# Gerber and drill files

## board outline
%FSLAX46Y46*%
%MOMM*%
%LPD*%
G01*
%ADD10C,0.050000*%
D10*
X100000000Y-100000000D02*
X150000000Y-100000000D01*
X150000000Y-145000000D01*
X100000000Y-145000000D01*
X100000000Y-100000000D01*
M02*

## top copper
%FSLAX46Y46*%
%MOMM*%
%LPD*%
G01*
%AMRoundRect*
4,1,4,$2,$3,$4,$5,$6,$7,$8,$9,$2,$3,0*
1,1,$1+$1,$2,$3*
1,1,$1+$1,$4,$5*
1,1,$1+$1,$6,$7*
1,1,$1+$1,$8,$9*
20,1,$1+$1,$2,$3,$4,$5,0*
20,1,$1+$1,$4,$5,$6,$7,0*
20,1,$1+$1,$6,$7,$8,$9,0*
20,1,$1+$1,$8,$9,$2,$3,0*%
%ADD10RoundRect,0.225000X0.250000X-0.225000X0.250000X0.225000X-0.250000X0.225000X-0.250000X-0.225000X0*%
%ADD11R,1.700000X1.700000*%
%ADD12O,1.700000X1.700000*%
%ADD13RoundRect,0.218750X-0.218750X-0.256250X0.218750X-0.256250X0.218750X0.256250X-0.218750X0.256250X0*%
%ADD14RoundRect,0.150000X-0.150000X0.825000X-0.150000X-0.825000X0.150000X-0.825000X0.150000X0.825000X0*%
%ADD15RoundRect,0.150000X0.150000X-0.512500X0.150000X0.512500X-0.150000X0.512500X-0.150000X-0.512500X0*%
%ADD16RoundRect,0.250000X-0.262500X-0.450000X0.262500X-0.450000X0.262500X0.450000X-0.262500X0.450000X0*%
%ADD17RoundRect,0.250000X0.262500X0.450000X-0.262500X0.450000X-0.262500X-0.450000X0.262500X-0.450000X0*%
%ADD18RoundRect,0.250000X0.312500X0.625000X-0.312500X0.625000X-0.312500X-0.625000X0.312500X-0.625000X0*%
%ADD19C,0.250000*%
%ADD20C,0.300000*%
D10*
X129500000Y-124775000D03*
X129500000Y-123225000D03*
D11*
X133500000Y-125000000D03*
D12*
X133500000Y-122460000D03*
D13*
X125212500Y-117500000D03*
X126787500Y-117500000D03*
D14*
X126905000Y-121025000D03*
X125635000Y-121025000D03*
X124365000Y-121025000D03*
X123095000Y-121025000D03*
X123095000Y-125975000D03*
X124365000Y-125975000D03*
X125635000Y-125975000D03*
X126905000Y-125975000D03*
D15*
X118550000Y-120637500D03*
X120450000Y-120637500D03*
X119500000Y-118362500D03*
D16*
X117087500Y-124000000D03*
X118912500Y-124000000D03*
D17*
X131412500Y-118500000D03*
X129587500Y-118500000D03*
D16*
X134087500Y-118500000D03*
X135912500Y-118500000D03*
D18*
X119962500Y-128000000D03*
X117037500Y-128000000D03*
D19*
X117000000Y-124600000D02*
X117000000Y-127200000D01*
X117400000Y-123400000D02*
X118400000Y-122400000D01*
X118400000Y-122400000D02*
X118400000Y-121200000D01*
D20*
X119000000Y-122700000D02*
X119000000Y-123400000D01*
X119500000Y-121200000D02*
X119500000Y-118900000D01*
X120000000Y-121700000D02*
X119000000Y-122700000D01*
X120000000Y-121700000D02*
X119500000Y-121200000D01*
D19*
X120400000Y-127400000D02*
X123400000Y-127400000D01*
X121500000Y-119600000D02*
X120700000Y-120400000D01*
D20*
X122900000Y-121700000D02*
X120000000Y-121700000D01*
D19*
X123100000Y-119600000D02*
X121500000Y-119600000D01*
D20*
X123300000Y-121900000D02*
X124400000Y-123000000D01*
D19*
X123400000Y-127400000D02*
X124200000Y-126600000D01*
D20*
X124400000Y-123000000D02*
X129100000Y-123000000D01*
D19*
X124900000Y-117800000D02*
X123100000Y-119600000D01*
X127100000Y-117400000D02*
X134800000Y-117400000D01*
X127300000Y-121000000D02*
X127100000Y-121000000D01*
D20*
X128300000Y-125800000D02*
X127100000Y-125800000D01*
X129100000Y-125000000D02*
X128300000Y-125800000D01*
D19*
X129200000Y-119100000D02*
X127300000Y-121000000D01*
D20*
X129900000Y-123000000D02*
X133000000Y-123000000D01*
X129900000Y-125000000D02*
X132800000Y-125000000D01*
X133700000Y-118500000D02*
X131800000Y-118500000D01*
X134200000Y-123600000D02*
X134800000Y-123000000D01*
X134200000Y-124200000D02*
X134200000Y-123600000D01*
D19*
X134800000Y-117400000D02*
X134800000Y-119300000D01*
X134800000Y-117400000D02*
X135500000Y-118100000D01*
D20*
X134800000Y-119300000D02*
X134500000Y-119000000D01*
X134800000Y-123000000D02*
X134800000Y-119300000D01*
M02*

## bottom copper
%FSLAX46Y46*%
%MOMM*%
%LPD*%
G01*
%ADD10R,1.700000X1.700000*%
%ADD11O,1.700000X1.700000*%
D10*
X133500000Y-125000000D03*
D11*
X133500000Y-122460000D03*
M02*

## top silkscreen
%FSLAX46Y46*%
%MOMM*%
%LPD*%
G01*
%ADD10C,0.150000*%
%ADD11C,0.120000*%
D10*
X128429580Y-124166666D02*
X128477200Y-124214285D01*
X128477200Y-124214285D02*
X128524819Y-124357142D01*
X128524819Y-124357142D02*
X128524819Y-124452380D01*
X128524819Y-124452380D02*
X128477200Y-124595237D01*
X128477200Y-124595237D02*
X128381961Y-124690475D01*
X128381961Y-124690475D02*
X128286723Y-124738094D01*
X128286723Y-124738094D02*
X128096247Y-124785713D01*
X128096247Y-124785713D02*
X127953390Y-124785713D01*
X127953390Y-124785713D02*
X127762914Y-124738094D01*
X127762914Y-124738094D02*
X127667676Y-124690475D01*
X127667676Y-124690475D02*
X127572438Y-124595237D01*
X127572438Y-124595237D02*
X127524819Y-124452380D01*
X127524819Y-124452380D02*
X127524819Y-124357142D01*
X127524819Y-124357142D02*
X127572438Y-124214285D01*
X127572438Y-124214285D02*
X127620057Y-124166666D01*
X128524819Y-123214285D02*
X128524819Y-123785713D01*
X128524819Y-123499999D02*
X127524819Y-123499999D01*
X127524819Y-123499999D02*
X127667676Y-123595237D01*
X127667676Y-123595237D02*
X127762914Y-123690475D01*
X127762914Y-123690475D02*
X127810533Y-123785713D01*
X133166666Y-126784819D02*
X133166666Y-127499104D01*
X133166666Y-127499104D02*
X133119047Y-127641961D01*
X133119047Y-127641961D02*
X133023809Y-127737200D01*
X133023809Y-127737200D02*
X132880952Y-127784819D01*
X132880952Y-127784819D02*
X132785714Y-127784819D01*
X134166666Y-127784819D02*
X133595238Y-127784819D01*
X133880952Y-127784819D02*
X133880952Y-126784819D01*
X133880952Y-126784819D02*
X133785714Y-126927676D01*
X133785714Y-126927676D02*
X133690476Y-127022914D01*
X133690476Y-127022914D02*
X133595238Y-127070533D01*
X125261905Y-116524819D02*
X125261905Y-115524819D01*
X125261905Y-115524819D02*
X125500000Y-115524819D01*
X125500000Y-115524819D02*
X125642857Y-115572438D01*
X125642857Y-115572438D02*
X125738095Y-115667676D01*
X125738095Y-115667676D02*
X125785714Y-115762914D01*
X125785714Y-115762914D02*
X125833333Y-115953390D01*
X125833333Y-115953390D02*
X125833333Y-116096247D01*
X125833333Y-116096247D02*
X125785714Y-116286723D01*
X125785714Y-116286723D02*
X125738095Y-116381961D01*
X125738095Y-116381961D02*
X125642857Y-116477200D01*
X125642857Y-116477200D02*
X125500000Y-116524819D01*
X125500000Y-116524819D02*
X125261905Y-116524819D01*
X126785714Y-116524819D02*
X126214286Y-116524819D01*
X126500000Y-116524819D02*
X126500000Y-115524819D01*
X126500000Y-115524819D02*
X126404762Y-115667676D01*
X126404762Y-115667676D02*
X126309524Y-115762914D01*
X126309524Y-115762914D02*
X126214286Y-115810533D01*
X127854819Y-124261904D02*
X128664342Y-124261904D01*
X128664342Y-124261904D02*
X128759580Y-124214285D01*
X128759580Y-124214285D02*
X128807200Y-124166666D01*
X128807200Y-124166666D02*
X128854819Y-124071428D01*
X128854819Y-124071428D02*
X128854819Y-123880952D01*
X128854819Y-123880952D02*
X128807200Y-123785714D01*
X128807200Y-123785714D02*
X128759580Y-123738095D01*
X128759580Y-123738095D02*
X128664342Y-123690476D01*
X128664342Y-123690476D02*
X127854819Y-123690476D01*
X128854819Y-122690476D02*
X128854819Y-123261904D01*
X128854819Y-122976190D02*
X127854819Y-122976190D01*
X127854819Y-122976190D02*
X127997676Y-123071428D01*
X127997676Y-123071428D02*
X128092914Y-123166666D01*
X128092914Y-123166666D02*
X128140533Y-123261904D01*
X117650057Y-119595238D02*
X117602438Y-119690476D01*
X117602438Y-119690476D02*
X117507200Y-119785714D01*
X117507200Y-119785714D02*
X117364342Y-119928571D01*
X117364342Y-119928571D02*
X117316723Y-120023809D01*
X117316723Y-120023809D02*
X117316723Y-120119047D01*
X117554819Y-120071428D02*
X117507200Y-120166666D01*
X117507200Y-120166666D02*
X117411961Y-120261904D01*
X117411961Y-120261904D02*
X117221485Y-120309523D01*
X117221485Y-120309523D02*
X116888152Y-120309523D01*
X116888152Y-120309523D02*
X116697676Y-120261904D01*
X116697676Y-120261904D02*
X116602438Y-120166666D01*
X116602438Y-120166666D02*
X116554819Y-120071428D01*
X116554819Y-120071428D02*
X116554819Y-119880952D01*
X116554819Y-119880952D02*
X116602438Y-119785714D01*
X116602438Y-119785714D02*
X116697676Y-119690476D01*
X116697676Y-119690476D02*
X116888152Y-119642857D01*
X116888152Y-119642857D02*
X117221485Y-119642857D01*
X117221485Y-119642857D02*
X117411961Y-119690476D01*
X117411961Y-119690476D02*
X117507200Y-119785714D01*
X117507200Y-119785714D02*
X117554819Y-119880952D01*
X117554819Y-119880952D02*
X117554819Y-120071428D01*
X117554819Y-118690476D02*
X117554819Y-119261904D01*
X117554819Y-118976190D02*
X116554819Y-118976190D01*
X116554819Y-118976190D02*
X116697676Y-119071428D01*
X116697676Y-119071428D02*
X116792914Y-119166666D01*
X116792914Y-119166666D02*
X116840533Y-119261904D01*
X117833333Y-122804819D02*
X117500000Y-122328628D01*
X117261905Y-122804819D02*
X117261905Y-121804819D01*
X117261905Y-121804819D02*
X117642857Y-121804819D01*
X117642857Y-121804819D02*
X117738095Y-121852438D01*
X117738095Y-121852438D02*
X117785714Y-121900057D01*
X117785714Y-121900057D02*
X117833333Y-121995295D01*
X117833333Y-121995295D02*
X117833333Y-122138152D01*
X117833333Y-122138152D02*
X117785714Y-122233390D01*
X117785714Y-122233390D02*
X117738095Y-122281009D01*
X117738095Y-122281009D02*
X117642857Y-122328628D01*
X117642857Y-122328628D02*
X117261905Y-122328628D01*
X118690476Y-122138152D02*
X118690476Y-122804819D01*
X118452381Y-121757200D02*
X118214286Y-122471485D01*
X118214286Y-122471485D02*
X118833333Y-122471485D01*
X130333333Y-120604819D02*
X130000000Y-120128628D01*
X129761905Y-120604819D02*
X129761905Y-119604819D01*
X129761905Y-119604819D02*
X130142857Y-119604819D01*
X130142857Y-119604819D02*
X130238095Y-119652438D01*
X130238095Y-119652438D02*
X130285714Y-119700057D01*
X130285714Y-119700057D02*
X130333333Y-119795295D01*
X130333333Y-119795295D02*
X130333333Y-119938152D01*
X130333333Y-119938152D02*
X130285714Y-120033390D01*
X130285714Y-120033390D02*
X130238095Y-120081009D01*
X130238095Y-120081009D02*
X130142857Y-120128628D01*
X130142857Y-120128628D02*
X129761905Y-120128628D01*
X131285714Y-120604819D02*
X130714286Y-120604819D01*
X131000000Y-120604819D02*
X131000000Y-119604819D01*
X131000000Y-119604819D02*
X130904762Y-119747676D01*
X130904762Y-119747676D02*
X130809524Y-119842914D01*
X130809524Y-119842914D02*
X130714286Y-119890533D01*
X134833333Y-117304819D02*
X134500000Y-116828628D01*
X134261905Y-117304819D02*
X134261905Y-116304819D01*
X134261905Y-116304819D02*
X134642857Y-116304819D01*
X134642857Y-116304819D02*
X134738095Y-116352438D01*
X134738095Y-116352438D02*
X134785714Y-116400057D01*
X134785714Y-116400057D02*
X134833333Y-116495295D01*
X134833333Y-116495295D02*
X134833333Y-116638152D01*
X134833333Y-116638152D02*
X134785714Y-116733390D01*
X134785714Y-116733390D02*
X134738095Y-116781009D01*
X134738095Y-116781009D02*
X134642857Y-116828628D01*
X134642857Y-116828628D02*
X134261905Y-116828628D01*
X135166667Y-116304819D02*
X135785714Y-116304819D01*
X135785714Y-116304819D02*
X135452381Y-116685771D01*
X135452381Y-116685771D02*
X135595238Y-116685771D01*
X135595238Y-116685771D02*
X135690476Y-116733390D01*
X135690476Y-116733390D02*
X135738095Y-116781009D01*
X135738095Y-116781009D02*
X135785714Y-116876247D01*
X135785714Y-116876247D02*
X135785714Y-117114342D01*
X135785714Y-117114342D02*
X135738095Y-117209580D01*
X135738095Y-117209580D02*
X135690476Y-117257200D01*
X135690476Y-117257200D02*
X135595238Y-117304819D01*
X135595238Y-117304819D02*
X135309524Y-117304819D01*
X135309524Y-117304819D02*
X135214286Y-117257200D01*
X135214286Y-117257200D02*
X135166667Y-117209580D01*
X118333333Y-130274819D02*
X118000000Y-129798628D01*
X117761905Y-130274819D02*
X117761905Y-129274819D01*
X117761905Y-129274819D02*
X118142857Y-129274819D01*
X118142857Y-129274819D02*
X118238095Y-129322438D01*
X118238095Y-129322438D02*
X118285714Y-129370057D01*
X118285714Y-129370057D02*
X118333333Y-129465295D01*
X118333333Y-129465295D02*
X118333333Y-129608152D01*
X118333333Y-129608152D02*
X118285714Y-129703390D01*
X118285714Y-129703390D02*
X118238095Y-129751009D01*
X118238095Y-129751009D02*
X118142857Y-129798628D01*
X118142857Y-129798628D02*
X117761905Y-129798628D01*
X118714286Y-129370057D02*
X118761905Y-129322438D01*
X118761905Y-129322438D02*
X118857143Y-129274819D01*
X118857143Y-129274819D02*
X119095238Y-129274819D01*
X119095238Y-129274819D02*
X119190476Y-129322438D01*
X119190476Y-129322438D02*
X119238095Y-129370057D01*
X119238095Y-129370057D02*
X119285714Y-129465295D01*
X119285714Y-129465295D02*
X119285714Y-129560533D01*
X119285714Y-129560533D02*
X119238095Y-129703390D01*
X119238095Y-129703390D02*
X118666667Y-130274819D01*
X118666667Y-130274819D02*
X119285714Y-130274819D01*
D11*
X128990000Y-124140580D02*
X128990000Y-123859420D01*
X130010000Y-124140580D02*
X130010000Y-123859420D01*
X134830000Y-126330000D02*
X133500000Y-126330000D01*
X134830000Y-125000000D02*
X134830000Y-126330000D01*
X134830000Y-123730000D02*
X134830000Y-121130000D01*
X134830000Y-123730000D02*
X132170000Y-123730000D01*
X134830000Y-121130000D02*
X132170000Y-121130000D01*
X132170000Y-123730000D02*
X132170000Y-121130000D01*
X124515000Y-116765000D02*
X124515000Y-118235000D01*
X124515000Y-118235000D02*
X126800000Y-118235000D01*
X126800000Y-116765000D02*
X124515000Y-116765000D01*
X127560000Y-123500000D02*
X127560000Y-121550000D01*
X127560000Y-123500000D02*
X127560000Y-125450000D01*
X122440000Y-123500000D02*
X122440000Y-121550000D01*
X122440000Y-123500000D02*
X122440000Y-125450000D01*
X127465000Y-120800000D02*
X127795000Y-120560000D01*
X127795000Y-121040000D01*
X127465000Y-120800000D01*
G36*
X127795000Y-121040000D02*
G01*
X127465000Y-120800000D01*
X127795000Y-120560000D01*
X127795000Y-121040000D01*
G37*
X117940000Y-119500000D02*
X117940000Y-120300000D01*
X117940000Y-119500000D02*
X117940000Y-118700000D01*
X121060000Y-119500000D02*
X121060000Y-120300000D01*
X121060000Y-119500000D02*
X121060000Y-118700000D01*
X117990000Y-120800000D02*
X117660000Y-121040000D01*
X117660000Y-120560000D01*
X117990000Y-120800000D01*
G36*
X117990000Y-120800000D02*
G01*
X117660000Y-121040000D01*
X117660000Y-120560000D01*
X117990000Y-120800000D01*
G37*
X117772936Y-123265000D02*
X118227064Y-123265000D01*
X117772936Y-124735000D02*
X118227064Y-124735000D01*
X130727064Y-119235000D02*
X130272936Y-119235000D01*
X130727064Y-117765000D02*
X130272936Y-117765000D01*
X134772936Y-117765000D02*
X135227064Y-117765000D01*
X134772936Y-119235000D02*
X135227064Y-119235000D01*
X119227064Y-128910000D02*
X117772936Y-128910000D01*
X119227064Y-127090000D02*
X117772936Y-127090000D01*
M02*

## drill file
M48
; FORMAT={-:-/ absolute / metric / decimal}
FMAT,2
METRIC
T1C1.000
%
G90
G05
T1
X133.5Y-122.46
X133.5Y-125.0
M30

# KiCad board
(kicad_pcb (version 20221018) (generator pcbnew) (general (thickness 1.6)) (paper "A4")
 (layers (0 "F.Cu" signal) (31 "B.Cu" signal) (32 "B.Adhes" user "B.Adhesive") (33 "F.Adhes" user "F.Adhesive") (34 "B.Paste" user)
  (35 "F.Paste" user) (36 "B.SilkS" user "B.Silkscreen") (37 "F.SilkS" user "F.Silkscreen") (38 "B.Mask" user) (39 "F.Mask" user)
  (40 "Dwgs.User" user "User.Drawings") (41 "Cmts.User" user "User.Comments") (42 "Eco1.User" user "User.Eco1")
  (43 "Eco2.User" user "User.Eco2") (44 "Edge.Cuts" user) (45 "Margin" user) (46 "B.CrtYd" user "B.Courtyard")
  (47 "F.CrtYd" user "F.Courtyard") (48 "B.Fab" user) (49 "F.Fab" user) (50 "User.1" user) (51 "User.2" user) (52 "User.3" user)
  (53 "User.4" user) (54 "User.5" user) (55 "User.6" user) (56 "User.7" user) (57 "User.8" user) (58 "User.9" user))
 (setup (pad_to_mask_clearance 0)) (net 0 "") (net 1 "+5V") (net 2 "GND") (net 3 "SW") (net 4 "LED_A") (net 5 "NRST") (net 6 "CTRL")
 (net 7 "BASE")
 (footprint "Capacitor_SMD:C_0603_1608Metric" (layer "F.Cu") (at 129.5 124 90)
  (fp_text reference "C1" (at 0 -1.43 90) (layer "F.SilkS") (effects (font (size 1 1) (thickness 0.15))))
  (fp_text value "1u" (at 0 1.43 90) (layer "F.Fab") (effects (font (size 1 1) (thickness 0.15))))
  (fp_line (start -0.14058 -0.51) (end 0.14058 -0.51) (stroke (width 0.12) (type solid)) (layer "F.SilkS"))
  (fp_line (start -0.14058 0.51) (end 0.14058 0.51) (stroke (width 0.12) (type solid)) (layer "F.SilkS"))
  (pad "1" smd roundrect (at -0.775 0 90) (size 0.9 0.95) (layers "F.Cu" "F.Paste" "F.Mask") (roundrect_rratio 0.25) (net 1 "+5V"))
  (pad "2" smd roundrect (at 0.775 0 90) (size 0.9 0.95) (layers "F.Cu" "F.Paste" "F.Mask") (roundrect_rratio 0.25) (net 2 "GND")))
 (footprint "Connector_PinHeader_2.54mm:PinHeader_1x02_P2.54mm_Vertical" (layer "F.Cu") (at 133.5 125 180)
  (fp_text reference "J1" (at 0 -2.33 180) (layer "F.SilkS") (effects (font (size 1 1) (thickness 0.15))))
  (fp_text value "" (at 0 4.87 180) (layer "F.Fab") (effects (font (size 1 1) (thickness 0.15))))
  (fp_line (start -1.33 -1.33) (end 0 -1.33) (stroke (width 0.12) (type solid)) (layer "F.SilkS"))
  (fp_line (start -1.33 0) (end -1.33 -1.33) (stroke (width 0.12) (type solid)) (layer "F.SilkS"))
  (fp_line (start -1.33 1.27) (end -1.33 3.87) (stroke (width 0.12) (type solid)) (layer "F.SilkS"))
  (fp_line (start -1.33 1.27) (end 1.33 1.27) (stroke (width 0.12) (type solid)) (layer "F.SilkS"))
  (fp_line (start -1.33 3.87) (end 1.33 3.87) (stroke (width 0.12) (type solid)) (layer "F.SilkS"))
  (fp_line (start 1.33 1.27) (end 1.33 3.87) (stroke (width 0.12) (type solid)) (layer "F.SilkS"))
  (pad "1" thru_hole rect (at 0 0 180) (size 1.7 1.7) (drill 1) (layers "*.Cu" "*.Mask") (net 1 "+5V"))
  (pad "2" thru_hole oval (at 0 2.54 180) (size 1.7 1.7) (drill 1) (layers "*.Cu" "*.Mask") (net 2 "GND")))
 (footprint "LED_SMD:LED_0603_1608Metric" (layer "F.Cu") (at 126 117.5)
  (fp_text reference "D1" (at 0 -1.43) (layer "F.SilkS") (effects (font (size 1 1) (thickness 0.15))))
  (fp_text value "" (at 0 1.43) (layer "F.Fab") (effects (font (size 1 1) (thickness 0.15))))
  (fp_line (start -1.485 -0.735) (end -1.485 0.735) (stroke (width 0.12) (type solid)) (layer "F.SilkS"))
  (fp_line (start -1.485 0.735) (end 0.8 0.735) (stroke (width 0.12) (type solid)) (layer "F.SilkS"))
  (fp_line (start 0.8 -0.735) (end -1.485 -0.735) (stroke (width 0.12) (type solid)) (layer "F.SilkS"))
  (pad "1" smd roundrect (at -0.7875 0) (size 0.875 0.95) (layers "F.Cu" "F.Paste" "F.Mask") (roundrect_rratio 0.25) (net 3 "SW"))
  (pad "2" smd roundrect (at 0.7875 0) (size 0.875 0.95) (layers "F.Cu" "F.Paste" "F.Mask") (roundrect_rratio 0.25) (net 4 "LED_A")))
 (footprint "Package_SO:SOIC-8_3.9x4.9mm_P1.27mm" (layer "F.Cu") (at 125 123.5 -90)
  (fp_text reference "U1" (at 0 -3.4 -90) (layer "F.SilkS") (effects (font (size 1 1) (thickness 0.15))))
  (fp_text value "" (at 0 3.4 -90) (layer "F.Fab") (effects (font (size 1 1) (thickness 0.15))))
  (fp_line (start 0 -2.56) (end -1.95 -2.56) (stroke (width 0.12) (type solid)) (layer "F.SilkS"))
  (fp_line (start 0 -2.56) (end 1.95 -2.56) (stroke (width 0.12) (type solid)) (layer "F.SilkS"))
  (fp_line (start 0 2.56) (end -1.95 2.56) (stroke (width 0.12) (type solid)) (layer "F.SilkS"))
  (fp_line (start 0 2.56) (end 1.95 2.56) (stroke (width 0.12) (type solid)) (layer "F.SilkS"))
  (fp_poly
   (pts (xy -2.7 -2.465) (xy -2.94 -2.795) (xy -2.46 -2.795) (xy -2.7 -2.465)) (stroke (width 0.12) (type solid)) (fill solid)
   (layer "F.SilkS"))
  (pad "1" smd roundrect (at -2.475 -1.905 270) (size 1.95 0.6) (layers "F.Cu" "F.Paste" "F.Mask") (roundrect_rratio 0.25) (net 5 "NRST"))
  (pad "2" smd roundrect (at -2.475 -0.635 270) (size 1.95 0.6) (layers "F.Cu" "F.Paste" "F.Mask") (roundrect_rratio 0.25))
  (pad "3" smd roundrect (at -2.475 0.635 270) (size 1.95 0.6) (layers "F.Cu" "F.Paste" "F.Mask") (roundrect_rratio 0.25))
  (pad "4" smd roundrect (at -2.475 1.905 270) (size 1.95 0.6) (layers "F.Cu" "F.Paste" "F.Mask") (roundrect_rratio 0.25) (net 2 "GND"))
  (pad "5" smd roundrect (at 2.475 1.905 270) (size 1.95 0.6) (layers "F.Cu" "F.Paste" "F.Mask") (roundrect_rratio 0.25))
  (pad "6" smd roundrect (at 2.475 0.635 270) (size 1.95 0.6) (layers "F.Cu" "F.Paste" "F.Mask") (roundrect_rratio 0.25) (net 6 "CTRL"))
  (pad "7" smd roundrect (at 2.475 -0.635 270) (size 1.95 0.6) (layers "F.Cu" "F.Paste" "F.Mask") (roundrect_rratio 0.25))
  (pad "8" smd roundrect (at 2.475 -1.905 270) (size 1.95 0.6) (layers "F.Cu" "F.Paste" "F.Mask") (roundrect_rratio 0.25) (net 1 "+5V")))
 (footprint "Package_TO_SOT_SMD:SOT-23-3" (layer "F.Cu") (at 119.5 119.5 90)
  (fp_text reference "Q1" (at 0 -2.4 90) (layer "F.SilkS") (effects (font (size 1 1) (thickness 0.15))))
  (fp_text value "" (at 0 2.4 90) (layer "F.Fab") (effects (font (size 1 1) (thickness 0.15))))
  (fp_line (start 0 -1.56) (end -0.8 -1.56) (stroke (width 0.12) (type solid)) (layer "F.SilkS"))
  (fp_line (start 0 -1.56) (end 0.8 -1.56) (stroke (width 0.12) (type solid)) (layer "F.SilkS"))
  (fp_line (start 0 1.56) (end -0.8 1.56) (stroke (width 0.12) (type solid)) (layer "F.SilkS"))
  (fp_line (start 0 1.56) (end 0.8 1.56) (stroke (width 0.12) (type solid)) (layer "F.SilkS"))
  (fp_poly
   (pts (xy -1.3 -1.51) (xy -1.54 -1.84) (xy -1.06 -1.84) (xy -1.3 -1.51)) (stroke (width 0.12) (type solid)) (fill solid) (layer "F.SilkS"))
  (pad "1" smd roundrect (at -1.1375 -0.95 90) (size 1.325 0.6) (layers "F.Cu" "F.Paste" "F.Mask") (roundrect_rratio 0.25) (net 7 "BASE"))
  (pad "2" smd roundrect (at -1.1375 0.95 90) (size 1.325 0.6) (layers "F.Cu" "F.Paste" "F.Mask") (roundrect_rratio 0.25) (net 3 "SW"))
  (pad "3" smd roundrect (at 1.1375 0 90) (size 1.325 0.6) (layers "F.Cu" "F.Paste" "F.Mask") (roundrect_rratio 0.25) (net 2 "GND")))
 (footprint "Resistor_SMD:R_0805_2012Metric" (layer "F.Cu") (at 118 124)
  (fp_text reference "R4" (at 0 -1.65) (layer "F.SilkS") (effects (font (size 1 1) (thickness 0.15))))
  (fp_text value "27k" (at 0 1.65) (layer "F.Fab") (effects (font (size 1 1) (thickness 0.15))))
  (fp_line (start -0.227064 -0.735) (end 0.227064 -0.735) (stroke (width 0.12) (type solid)) (layer "F.SilkS"))
  (fp_line (start -0.227064 0.735) (end 0.227064 0.735) (stroke (width 0.12) (type solid)) (layer "F.SilkS"))
  (pad "1" smd roundrect (at -0.9125 0) (size 1.025 1.4) (layers "F.Cu" "F.Paste" "F.Mask") (roundrect_rratio 0.243902) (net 7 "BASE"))
  (pad "2" smd roundrect (at 0.9125 0) (size 1.025 1.4) (layers "F.Cu" "F.Paste" "F.Mask") (roundrect_rratio 0.243902) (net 2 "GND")))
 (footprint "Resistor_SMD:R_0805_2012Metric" (layer "F.Cu") (at 130.5 118.5 180)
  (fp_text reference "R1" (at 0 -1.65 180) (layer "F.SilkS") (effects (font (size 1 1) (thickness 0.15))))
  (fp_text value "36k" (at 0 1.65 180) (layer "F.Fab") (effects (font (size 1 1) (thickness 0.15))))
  (fp_line (start -0.227064 -0.735) (end 0.227064 -0.735) (stroke (width 0.12) (type solid)) (layer "F.SilkS"))
  (fp_line (start -0.227064 0.735) (end 0.227064 0.735) (stroke (width 0.12) (type solid)) (layer "F.SilkS"))
  (pad "1" smd roundrect (at -0.9125 0 180) (size 1.025 1.4) (layers "F.Cu" "F.Paste" "F.Mask") (roundrect_rratio 0.243902) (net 1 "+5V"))
  (pad "2" smd roundrect (at 0.9125 0 180) (size 1.025 1.4) (layers "F.Cu" "F.Paste" "F.Mask") (roundrect_rratio 0.243902) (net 5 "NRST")))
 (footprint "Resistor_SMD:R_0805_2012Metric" (layer "F.Cu") (at 135 118.5)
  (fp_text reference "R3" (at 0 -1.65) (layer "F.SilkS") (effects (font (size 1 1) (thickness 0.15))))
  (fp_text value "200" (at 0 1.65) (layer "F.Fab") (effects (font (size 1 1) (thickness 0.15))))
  (fp_line (start -0.227064 -0.735) (end 0.227064 -0.735) (stroke (width 0.12) (type solid)) (layer "F.SilkS"))
  (fp_line (start -0.227064 0.735) (end 0.227064 0.735) (stroke (width 0.12) (type solid)) (layer "F.SilkS"))
  (pad "1" smd roundrect (at -0.9125 0) (size 1.025 1.4) (layers "F.Cu" "F.Paste" "F.Mask") (roundrect_rratio 0.243902) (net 1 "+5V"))
  (pad "2" smd roundrect (at 0.9125 0) (size 1.025 1.4) (layers "F.Cu" "F.Paste" "F.Mask") (roundrect_rratio 0.243902) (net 4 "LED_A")))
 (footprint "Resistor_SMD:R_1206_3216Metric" (layer "F.Cu") (at 118.5 128 180)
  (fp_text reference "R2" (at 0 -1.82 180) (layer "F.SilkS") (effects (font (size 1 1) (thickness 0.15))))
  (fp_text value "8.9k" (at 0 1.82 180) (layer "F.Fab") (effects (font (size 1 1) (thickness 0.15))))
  (fp_line (start -0.727064 -0.91) (end 0.727064 -0.91) (stroke (width 0.12) (type solid)) (layer "F.SilkS"))
  (fp_line (start -0.727064 0.91) (end 0.727064 0.91) (stroke (width 0.12) (type solid)) (layer "F.SilkS"))
  (pad "1" smd roundrect (at -1.4625 0 180) (size 1.125 1.75) (layers "F.Cu" "F.Paste" "F.Mask") (roundrect_rratio 0.222222) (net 6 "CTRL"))
  (pad "2" smd roundrect (at 1.4625 0 180) (size 1.125 1.75) (layers "F.Cu" "F.Paste" "F.Mask") (roundrect_rratio 0.222222) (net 7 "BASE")))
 (gr_rect (start 100 100) (end 150 145) (stroke (width 0.05) (type default)) (fill none) (layer "Edge.Cuts"))
 (segment (start 117 124.6) (end 117 127.2) (width 0.25) (layer "F.Cu") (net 7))
 (segment (start 117.4 123.4) (end 118.4 122.4) (width 0.25) (layer "F.Cu") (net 7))
 (segment (start 118.4 122.4) (end 118.4 121.2) (width 0.25) (layer "F.Cu") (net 7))
 (segment (start 119 122.7) (end 119 123.4) (width 0.3) (layer "F.Cu") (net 2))
 (segment (start 119.5 121.2) (end 119.5 118.9) (width 0.3) (layer "F.Cu") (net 2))
 (segment (start 120 121.7) (end 119 122.7) (width 0.3) (layer "F.Cu") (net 2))
 (segment (start 120 121.7) (end 119.5 121.2) (width 0.3) (layer "F.Cu") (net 2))
 (segment (start 120.4 127.4) (end 123.4 127.4) (width 0.25) (layer "F.Cu") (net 6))
 (segment (start 121.5 119.6) (end 120.7 120.4) (width 0.25) (layer "F.Cu") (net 3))
 (segment (start 122.9 121.7) (end 120 121.7) (width 0.3) (layer "F.Cu") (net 2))
 (segment (start 123.1 119.6) (end 121.5 119.6) (width 0.25) (layer "F.Cu") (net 3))
 (segment (start 123.3 121.9) (end 124.4 123) (width 0.3) (layer "F.Cu") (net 2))
 (segment (start 123.4 127.4) (end 124.2 126.6) (width 0.25) (layer "F.Cu") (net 6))
 (segment (start 124.4 123) (end 129.1 123) (width 0.3) (layer "F.Cu") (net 2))
 (segment (start 124.9 117.8) (end 123.1 119.6) (width 0.25) (layer "F.Cu") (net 3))
 (segment (start 127.1 117.4) (end 134.8 117.4) (width 0.25) (layer "F.Cu") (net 4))
 (segment (start 127.3 121) (end 127.1 121) (width 0.25) (layer "F.Cu") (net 5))
 (segment (start 128.3 125.8) (end 127.1 125.8) (width 0.3) (layer "F.Cu") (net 1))
 (segment (start 129.1 125) (end 128.3 125.8) (width 0.3) (layer "F.Cu") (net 1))
 (segment (start 129.2 119.1) (end 127.3 121) (width 0.25) (layer "F.Cu") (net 5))
 (segment (start 129.9 123) (end 133 123) (width 0.3) (layer "F.Cu") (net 2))
 (segment (start 129.9 125) (end 132.8 125) (width 0.3) (layer "F.Cu") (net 1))
 (segment (start 133.7 118.5) (end 131.8 118.5) (width 0.3) (layer "F.Cu") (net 1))
 (segment (start 134.2 123.6) (end 134.8 123) (width 0.3) (layer "F.Cu") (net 1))
 (segment (start 134.2 124.2) (end 134.2 123.6) (width 0.3) (layer "F.Cu") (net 1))
 (segment (start 134.8 117.4) (end 134.8 119.3) (width 0.25) (layer "F.Cu") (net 4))
 (segment (start 134.8 117.4) (end 135.5 118.1) (width 0.25) (layer "F.Cu") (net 4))
 (segment (start 134.8 119.3) (end 134.5 119) (width 0.3) (layer "F.Cu") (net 1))
 (segment (start 134.8 123) (end 134.8 119.3) (width 0.3) (layer "F.Cu") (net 1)))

